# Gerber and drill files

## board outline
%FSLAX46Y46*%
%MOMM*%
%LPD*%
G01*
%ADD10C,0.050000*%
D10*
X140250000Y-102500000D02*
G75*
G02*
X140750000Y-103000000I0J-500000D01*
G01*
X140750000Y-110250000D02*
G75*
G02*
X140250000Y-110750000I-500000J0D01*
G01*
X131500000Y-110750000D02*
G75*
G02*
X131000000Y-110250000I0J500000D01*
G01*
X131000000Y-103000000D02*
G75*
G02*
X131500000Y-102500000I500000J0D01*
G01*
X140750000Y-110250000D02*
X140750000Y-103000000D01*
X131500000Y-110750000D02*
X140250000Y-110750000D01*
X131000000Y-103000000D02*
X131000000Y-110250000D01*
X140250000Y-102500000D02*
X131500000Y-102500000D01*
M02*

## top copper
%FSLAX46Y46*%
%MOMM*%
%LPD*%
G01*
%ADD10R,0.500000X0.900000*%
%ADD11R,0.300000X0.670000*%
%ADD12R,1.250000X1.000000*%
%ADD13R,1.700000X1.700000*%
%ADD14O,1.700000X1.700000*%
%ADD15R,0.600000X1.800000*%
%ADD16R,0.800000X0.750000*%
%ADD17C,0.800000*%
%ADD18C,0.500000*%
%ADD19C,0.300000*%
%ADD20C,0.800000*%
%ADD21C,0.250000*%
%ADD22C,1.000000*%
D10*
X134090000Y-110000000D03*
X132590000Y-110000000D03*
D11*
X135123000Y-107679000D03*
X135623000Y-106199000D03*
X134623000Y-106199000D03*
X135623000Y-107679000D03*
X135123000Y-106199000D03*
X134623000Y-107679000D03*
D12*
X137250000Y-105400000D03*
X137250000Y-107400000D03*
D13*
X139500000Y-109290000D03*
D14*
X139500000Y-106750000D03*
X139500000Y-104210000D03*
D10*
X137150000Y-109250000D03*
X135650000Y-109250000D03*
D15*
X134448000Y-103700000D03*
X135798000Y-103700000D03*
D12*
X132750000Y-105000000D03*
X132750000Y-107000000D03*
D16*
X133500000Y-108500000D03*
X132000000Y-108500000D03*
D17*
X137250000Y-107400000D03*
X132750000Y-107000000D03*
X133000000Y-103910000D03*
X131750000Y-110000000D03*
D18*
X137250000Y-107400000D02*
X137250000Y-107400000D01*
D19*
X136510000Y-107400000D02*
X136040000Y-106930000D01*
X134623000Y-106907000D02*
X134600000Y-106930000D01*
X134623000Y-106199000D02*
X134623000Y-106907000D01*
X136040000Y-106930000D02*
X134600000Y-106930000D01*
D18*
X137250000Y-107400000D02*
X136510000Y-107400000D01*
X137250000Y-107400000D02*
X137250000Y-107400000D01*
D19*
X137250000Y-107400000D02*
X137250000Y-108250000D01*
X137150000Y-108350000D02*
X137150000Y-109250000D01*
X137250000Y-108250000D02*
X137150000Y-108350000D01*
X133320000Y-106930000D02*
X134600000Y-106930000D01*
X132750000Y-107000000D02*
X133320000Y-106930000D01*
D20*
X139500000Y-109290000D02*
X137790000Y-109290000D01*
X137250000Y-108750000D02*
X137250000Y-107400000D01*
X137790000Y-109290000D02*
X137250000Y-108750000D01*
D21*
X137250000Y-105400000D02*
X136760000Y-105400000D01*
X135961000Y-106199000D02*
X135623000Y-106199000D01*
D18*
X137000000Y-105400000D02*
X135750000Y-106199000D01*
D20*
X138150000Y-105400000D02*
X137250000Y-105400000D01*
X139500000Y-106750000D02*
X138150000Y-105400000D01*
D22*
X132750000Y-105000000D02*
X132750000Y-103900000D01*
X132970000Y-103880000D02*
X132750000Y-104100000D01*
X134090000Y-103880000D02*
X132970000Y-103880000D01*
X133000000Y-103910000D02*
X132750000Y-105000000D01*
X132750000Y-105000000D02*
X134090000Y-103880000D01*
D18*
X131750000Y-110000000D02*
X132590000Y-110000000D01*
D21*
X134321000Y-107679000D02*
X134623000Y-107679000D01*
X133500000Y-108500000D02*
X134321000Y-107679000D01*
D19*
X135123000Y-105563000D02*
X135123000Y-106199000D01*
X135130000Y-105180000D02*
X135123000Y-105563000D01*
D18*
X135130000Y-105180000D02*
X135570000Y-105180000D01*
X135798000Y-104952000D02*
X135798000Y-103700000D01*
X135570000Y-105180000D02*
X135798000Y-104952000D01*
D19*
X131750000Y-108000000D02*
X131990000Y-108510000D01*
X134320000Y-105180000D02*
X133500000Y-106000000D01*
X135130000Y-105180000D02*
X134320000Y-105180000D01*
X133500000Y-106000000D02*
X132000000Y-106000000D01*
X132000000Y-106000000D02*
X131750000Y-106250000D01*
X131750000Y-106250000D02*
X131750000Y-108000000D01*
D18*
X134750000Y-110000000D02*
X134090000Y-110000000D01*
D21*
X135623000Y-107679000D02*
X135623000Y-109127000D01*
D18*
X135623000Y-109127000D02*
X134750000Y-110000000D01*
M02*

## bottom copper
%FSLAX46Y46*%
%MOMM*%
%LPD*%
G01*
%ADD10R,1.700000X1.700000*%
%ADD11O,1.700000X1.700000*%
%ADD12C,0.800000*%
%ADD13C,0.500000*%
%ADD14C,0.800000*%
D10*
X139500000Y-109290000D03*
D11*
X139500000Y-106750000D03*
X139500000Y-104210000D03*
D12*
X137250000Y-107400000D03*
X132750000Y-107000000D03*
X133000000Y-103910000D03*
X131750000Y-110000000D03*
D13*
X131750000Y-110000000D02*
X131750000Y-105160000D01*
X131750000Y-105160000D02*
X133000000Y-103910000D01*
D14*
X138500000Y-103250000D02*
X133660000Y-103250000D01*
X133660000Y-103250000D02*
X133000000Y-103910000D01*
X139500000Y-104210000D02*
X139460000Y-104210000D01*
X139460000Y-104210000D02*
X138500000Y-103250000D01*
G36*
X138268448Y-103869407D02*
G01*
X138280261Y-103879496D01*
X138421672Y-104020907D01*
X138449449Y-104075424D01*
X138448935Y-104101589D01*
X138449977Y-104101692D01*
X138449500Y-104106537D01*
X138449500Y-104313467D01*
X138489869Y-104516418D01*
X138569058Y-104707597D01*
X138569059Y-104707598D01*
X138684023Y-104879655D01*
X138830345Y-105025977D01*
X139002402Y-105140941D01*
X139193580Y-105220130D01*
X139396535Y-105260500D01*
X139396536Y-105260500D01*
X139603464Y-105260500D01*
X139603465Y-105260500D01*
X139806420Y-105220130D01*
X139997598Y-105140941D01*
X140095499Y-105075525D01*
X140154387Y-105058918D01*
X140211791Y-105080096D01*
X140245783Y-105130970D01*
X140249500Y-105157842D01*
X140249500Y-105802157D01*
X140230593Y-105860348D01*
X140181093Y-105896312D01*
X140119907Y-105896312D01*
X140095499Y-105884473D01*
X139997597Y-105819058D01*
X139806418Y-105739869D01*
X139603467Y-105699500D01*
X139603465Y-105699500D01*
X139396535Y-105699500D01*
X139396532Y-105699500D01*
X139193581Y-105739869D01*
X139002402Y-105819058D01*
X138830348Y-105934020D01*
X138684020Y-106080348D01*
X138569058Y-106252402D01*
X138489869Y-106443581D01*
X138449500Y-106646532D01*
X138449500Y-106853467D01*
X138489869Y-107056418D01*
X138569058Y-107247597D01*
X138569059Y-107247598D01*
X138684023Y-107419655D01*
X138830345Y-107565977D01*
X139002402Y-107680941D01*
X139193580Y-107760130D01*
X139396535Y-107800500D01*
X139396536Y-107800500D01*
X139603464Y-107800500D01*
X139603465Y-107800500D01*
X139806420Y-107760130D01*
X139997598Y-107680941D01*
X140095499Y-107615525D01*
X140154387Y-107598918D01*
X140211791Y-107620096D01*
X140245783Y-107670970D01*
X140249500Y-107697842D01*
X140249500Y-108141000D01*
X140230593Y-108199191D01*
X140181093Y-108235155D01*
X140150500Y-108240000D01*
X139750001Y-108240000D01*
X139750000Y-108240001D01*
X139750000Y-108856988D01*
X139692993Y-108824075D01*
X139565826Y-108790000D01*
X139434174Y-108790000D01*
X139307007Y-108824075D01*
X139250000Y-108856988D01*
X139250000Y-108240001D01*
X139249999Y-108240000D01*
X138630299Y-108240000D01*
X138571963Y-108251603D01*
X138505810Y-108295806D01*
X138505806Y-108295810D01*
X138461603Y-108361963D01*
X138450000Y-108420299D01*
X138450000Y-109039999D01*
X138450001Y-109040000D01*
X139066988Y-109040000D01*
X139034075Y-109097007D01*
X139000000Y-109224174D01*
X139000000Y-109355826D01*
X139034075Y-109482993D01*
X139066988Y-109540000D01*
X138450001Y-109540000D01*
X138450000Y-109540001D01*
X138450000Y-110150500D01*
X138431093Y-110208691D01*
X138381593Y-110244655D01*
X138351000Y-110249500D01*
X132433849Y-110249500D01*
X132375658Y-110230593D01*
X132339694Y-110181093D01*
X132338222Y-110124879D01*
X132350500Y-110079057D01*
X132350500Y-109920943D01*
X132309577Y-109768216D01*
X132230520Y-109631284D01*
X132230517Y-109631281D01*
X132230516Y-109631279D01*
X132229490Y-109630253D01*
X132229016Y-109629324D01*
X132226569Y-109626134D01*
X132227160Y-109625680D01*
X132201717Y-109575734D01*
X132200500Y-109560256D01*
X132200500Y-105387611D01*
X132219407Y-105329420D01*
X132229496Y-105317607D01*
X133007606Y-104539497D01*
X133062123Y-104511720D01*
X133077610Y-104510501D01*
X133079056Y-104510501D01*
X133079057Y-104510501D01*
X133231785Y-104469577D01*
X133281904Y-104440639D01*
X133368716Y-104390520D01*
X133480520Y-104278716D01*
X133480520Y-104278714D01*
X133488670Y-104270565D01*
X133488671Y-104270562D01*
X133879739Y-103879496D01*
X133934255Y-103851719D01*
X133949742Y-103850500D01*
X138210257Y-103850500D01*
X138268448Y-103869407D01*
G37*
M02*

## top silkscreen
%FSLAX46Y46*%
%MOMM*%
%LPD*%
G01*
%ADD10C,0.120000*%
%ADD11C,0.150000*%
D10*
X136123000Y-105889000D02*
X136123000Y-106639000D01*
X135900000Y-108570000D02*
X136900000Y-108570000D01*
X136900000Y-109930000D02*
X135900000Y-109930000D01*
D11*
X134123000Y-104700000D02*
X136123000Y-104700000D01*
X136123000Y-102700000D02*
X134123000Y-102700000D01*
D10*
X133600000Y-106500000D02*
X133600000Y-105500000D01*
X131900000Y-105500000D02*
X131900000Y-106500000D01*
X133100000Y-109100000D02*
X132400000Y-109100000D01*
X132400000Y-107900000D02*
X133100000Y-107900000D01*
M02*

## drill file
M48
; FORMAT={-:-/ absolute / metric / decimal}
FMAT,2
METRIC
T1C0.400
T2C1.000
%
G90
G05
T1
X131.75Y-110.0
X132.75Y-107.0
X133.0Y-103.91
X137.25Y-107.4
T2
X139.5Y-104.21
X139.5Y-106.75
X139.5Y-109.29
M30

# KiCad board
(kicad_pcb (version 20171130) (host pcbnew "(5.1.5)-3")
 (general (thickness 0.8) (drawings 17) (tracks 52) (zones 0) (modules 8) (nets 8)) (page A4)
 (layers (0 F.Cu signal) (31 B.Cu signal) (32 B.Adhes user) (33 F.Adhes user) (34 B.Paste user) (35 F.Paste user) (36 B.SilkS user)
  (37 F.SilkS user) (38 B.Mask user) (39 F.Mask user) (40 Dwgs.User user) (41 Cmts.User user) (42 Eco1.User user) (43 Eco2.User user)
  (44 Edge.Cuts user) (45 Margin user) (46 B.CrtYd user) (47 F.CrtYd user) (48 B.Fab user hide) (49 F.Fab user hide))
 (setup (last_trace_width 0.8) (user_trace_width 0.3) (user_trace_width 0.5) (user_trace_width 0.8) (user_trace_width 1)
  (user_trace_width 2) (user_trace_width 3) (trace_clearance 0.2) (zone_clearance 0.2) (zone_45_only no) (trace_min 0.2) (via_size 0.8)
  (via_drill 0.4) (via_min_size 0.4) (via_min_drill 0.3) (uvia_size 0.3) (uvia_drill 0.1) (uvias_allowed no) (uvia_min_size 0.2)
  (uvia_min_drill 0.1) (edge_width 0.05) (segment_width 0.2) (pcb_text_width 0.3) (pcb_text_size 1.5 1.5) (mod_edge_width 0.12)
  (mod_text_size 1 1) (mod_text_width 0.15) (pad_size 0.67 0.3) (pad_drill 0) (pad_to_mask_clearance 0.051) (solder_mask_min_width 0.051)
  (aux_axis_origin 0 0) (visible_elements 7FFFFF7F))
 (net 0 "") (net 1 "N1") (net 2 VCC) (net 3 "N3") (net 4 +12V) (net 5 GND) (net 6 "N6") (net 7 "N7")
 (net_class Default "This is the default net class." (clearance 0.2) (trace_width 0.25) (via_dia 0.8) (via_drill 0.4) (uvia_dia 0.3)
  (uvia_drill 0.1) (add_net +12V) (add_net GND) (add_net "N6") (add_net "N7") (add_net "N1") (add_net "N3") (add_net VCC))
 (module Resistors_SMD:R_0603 (layer F.Cu) (at 133.34 110 180)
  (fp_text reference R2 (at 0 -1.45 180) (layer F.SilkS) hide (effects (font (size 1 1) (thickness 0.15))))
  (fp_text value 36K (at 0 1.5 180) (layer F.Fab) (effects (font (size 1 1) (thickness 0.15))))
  (pad 1 smd rect (at -0.75 0 180) (size 0.5 0.9) (layers F.Cu F.Paste F.Mask) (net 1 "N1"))
  (pad 2 smd rect (at 0.75 0 180) (size 0.5 0.9) (layers F.Cu F.Paste F.Mask) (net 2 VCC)))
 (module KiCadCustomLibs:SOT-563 (layer F.Cu) (at 135.123 106.939 270)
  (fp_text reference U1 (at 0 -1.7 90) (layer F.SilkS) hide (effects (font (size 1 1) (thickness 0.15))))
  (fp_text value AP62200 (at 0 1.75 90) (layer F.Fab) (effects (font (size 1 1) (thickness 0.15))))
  (fp_line (start -1.05 -1) (end -0.3 -1) (layer F.SilkS) (width 0.12))
  (pad 5 smd rect (at 0.74 0 270) (size 0.67 0.3) (layers F.Cu F.Paste F.Mask) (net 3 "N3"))
  (pad 1 smd rect (at -0.74 -0.5 270) (size 0.67 0.3) (layers F.Cu F.Paste F.Mask) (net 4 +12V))
  (pad 3 smd rect (at -0.74 0.5 270) (size 0.67 0.3) (layers F.Cu F.Paste F.Mask) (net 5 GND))
  (pad 6 smd rect (at 0.74 -0.5 270) (size 0.67 0.3) (layers F.Cu F.Paste F.Mask) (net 1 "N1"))
  (pad 2 smd rect (at -0.74 0 270) (size 0.67 0.3) (layers F.Cu F.Paste F.Mask) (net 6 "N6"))
  (pad 4 smd rect (at 0.74 0.5 270) (size 0.67 0.3) (layers F.Cu F.Paste F.Mask) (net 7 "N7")))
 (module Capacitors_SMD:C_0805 (layer F.Cu) (at 137.25 106.4 270)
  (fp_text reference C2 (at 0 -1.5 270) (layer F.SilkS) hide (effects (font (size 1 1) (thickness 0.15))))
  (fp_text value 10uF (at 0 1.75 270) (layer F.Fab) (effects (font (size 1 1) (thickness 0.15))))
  (pad 1 smd rect (at -1 0 270) (size 1 1.25) (layers F.Cu F.Paste F.Mask) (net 4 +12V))
  (pad 2 smd rect (at 1 0 270) (size 1 1.25) (layers F.Cu F.Paste F.Mask) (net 5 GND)))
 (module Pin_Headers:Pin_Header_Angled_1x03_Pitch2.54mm (layer B.Cu) (at 139.5 109.29)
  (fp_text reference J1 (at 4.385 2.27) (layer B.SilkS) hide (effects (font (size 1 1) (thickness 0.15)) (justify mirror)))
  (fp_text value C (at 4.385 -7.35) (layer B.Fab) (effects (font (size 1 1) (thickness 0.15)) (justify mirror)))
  (pad 1 thru_hole rect (at 0 0) (size 1.7 1.7) (drill 1) (layers *.Cu *.Mask) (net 5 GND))
  (pad 2 thru_hole oval (at 0 -2.54) (size 1.7 1.7) (drill 1) (layers *.Cu *.Mask) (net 4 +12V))
  (pad 3 thru_hole oval (at 0 -5.08) (size 1.7 1.7) (drill 1) (layers *.Cu *.Mask) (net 2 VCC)))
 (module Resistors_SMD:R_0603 (layer F.Cu) (at 136.4 109.25 180)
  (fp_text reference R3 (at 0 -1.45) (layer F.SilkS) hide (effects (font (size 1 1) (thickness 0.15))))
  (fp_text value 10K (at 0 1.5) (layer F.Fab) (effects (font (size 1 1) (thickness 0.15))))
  (fp_line (start 0.5 0.68) (end -0.5 0.68) (layer F.SilkS) (width 0.12))
  (fp_line (start -0.5 -0.68) (end 0.5 -0.68) (layer F.SilkS) (width 0.12))
  (pad 1 smd rect (at -0.75 0 180) (size 0.5 0.9) (layers F.Cu F.Paste F.Mask) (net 5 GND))
  (pad 2 smd rect (at 0.75 0 180) (size 0.5 0.9) (layers F.Cu F.Paste F.Mask) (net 1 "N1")))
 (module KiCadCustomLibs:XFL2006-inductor (layer F.Cu) (at 135.123 103.7 180)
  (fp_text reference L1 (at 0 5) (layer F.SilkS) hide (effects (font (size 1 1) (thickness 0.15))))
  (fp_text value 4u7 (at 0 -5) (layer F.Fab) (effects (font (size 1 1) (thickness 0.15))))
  (fp_line (start 1 -1) (end -1 -1) (layer F.SilkS) (width 0.15))
  (fp_line (start -1 1) (end 1 1) (layer F.SilkS) (width 0.15))
  (pad 2 smd rect (at 0.675 0 180) (size 0.6 1.8) (layers F.Cu F.Paste F.Mask) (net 2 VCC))
  (pad 1 smd rect (at -0.675 0 180) (size 0.6 1.8) (layers F.Cu F.Paste F.Mask) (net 6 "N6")))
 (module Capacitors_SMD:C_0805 (layer F.Cu) (at 132.75 106 270)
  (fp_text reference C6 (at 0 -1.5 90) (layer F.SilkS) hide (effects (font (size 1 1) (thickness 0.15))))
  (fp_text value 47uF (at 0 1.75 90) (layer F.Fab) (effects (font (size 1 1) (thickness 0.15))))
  (fp_line (start 0.5 -0.85) (end -0.5 -0.85) (layer F.SilkS) (width 0.12))
  (fp_line (start -0.5 0.85) (end 0.5 0.85) (layer F.SilkS) (width 0.12))
  (pad 1 smd rect (at -1 0 270) (size 1 1.25) (layers F.Cu F.Paste F.Mask) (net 2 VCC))
  (pad 2 smd rect (at 1 0 270) (size 1 1.25) (layers F.Cu F.Paste F.Mask) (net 5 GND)))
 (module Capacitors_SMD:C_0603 (layer F.Cu) (at 132.75 108.5)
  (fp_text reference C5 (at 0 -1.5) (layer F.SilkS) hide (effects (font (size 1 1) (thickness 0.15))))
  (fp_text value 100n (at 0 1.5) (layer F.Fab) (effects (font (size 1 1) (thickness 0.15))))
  (fp_line (start 0.35 0.6) (end -0.35 0.6) (layer F.SilkS) (width 0.12))
  (fp_line (start -0.35 -0.6) (end 0.35 -0.6) (layer F.SilkS) (width 0.12))
  (pad 2 smd rect (at 0.75 0) (size 0.8 0.75) (layers F.Cu F.Paste F.Mask) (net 7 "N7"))
  (pad 1 smd rect (at -0.75 0) (size 0.8 0.75) (layers F.Cu F.Paste F.Mask) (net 6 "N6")))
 (gr_arc (start 140.25 103) (end 140.75 103) (angle -90) (layer Edge.Cuts) (width 0.05))
 (gr_arc (start 140.25 110.25) (end 140.25 110.75) (angle -90) (layer Edge.Cuts) (width 0.05))
 (gr_arc (start 131.5 110.25) (end 131 110.25) (angle -90) (layer Edge.Cuts) (width 0.05))
 (gr_arc (start 131.5 103) (end 131.5 102.5) (angle -90) (layer Edge.Cuts) (width 0.05))
 (gr_line (start 140.75 110.25) (end 140.75 103) (layer Edge.Cuts) (width 0.05))
 (gr_line (start 131.5 110.75) (end 140.25 110.75) (layer Edge.Cuts) (width 0.05))
 (gr_line (start 131 103) (end 131 110.25) (layer Edge.Cuts) (width 0.05))
 (gr_line (start 140.25 102.5) (end 131.5 102.5) (layer Edge.Cuts) (width 0.05))
 (segment (start 137.25 107.4) (end 137.25 107.4) (width 0.5) (layer F.Cu) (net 5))
 (segment (start 136.51 107.4) (end 136.04 106.93) (width 0.3) (layer F.Cu) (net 5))
 (segment (start 134.623 106.907) (end 134.6 106.93) (width 0.3) (layer F.Cu) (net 5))
 (segment (start 134.623 106.199) (end 134.623 106.907) (width 0.3) (layer F.Cu) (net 5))
 (segment (start 136.04 106.93) (end 134.6 106.93) (width 0.3) (layer F.Cu) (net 5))
 (segment (start 137.25 107.4) (end 136.51 107.4) (width 0.5) (layer F.Cu) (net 5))
 (segment (start 137.25 107.4) (end 137.25 107.4) (width 0.5) (layer F.Cu) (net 5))
 (via (at 137.25 107.4) (size 0.8) (drill 0.4) (layers F.Cu B.Cu) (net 5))
 (segment (start 137.25 107.4) (end 137.25 108.25) (width 0.3) (layer F.Cu) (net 5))
 (segment (start 137.15 108.35) (end 137.15 109.25) (width 0.3) (layer F.Cu) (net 5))
 (segment (start 137.25 108.25) (end 137.15 108.35) (width 0.3) (layer F.Cu) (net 5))
 (segment (start 133.32 106.93) (end 134.6 106.93) (width 0.3) (layer F.Cu) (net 5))
 (via (at 132.75 107) (size 0.8) (drill 0.4) (layers F.Cu B.Cu) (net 5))
 (segment (start 132.75 107) (end 133.32 106.93) (width 0.3) (layer F.Cu) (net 5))
 (segment (start 139.5 109.29) (end 137.79 109.29) (width 0.8) (layer F.Cu) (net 5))
 (segment (start 137.25 108.75) (end 137.25 107.4) (width 0.8) (layer F.Cu) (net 5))
 (segment (start 137.79 109.29) (end 137.25 108.75) (width 0.8) (layer F.Cu) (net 5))
 (segment (start 137.25 105.4) (end 136.76 105.4) (width 0.25) (layer F.Cu) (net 4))
 (segment (start 135.961 106.199) (end 135.623 106.199) (width 0.25) (layer F.Cu) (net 4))
 (segment (start 137 105.4) (end 135.75 106.199) (width 0.5) (layer F.Cu) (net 4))
 (segment (start 138.15 105.4) (end 137.25 105.4) (width 0.8) (layer F.Cu) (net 4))
 (segment (start 139.5 106.75) (end 138.15 105.4) (width 0.8) (layer F.Cu) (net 4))
 (via (at 133 103.91) (size 0.8) (drill 0.4) (layers F.Cu B.Cu) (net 2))
 (segment (start 132.75 105) (end 132.75 103.9) (width 1) (layer F.Cu) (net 2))
 (segment (start 132.97 103.88) (end 132.75 104.1) (width 1) (layer F.Cu) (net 2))
 (segment (start 134.09 103.88) (end 132.97 103.88) (width 1) (layer F.Cu) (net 2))
 (segment (start 133 103.91) (end 132.75 105) (width 1) (layer F.Cu) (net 2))
 (segment (start 132.75 105) (end 134.09 103.88) (width 1) (layer F.Cu) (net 2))
 (segment (start 131.75 110) (end 131.75 105.16) (width 0.5) (layer B.Cu) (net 2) (status 1000000))
 (segment (start 131.75 110) (end 132.59 110) (width 0.5) (layer F.Cu) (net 2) (status 1000000))
 (segment (start 131.75 105.16) (end 133 103.91) (width 0.5) (layer B.Cu) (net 2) (status 1000000))
 (via (at 131.75 110) (size 0.8) (drill 0.4) (layers F.Cu B.Cu) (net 2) (status 1000000))
 (segment (start 138.5 103.25) (end 133.66 103.25) (width 0.8) (layer B.Cu) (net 2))
 (segment (start 133.66 103.25) (end 133 103.91) (width 0.8) (layer B.Cu) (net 2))
 (segment (start 139.5 104.21) (end 139.46 104.21) (width 0.8) (layer B.Cu) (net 2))
 (segment (start 139.46 104.21) (end 138.5 103.25) (width 0.8) (layer B.Cu) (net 2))
 (segment (start 134.321 107.679) (end 134.623 107.679) (width 0.25) (layer F.Cu) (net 7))
 (segment (start 133.5 108.5) (end 134.321 107.679) (width 0.25) (layer F.Cu) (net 7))
 (segment (start 135.123 105.563) (end 135.123 106.199) (width 0.3) (layer F.Cu) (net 6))
 (segment (start 135.13 105.18) (end 135.123 105.563) (width 0.3) (layer F.Cu) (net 6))
 (segment (start 135.13 105.18) (end 135.57 105.18) (width 0.5) (layer F.Cu) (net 6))
 (segment (start 135.798 104.952) (end 135.798 103.7) (width 0.5) (layer F.Cu) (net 6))
 (segment (start 135.57 105.18) (end 135.798 104.952) (width 0.5) (layer F.Cu) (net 6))
 (segment (start 131.75 108) (end 131.99 108.51) (width 0.3) (layer F.Cu) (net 6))
 (segment (start 134.32 105.18) (end 133.5 106) (width 0.3) (layer F.Cu) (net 6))
 (segment (start 135.13 105.18) (end 134.32 105.18) (width 0.3) (layer F.Cu) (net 6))
 (segment (start 133.5 106) (end 132 106) (width 0.3) (layer F.Cu) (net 6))
 (segment (start 132 106) (end 131.75 106.25) (width 0.3) (layer F.Cu) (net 6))
 (segment (start 131.75 106.25) (end 131.75 108) (width 0.3) (layer F.Cu) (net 6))
 (segment (start 134.75 110) (end 134.09 110) (width 0.5) (layer F.Cu) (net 1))
 (segment (start 135.623 107.679) (end 135.623 109.127) (width 0.25) (layer F.Cu) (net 1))
 (segment (start 135.623 109.127) (end 134.75 110) (width 0.5) (layer F.Cu) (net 1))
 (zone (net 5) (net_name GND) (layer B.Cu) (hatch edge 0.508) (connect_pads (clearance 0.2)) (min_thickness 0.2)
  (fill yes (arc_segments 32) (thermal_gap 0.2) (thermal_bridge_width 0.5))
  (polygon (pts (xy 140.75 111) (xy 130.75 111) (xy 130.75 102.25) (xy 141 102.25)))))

